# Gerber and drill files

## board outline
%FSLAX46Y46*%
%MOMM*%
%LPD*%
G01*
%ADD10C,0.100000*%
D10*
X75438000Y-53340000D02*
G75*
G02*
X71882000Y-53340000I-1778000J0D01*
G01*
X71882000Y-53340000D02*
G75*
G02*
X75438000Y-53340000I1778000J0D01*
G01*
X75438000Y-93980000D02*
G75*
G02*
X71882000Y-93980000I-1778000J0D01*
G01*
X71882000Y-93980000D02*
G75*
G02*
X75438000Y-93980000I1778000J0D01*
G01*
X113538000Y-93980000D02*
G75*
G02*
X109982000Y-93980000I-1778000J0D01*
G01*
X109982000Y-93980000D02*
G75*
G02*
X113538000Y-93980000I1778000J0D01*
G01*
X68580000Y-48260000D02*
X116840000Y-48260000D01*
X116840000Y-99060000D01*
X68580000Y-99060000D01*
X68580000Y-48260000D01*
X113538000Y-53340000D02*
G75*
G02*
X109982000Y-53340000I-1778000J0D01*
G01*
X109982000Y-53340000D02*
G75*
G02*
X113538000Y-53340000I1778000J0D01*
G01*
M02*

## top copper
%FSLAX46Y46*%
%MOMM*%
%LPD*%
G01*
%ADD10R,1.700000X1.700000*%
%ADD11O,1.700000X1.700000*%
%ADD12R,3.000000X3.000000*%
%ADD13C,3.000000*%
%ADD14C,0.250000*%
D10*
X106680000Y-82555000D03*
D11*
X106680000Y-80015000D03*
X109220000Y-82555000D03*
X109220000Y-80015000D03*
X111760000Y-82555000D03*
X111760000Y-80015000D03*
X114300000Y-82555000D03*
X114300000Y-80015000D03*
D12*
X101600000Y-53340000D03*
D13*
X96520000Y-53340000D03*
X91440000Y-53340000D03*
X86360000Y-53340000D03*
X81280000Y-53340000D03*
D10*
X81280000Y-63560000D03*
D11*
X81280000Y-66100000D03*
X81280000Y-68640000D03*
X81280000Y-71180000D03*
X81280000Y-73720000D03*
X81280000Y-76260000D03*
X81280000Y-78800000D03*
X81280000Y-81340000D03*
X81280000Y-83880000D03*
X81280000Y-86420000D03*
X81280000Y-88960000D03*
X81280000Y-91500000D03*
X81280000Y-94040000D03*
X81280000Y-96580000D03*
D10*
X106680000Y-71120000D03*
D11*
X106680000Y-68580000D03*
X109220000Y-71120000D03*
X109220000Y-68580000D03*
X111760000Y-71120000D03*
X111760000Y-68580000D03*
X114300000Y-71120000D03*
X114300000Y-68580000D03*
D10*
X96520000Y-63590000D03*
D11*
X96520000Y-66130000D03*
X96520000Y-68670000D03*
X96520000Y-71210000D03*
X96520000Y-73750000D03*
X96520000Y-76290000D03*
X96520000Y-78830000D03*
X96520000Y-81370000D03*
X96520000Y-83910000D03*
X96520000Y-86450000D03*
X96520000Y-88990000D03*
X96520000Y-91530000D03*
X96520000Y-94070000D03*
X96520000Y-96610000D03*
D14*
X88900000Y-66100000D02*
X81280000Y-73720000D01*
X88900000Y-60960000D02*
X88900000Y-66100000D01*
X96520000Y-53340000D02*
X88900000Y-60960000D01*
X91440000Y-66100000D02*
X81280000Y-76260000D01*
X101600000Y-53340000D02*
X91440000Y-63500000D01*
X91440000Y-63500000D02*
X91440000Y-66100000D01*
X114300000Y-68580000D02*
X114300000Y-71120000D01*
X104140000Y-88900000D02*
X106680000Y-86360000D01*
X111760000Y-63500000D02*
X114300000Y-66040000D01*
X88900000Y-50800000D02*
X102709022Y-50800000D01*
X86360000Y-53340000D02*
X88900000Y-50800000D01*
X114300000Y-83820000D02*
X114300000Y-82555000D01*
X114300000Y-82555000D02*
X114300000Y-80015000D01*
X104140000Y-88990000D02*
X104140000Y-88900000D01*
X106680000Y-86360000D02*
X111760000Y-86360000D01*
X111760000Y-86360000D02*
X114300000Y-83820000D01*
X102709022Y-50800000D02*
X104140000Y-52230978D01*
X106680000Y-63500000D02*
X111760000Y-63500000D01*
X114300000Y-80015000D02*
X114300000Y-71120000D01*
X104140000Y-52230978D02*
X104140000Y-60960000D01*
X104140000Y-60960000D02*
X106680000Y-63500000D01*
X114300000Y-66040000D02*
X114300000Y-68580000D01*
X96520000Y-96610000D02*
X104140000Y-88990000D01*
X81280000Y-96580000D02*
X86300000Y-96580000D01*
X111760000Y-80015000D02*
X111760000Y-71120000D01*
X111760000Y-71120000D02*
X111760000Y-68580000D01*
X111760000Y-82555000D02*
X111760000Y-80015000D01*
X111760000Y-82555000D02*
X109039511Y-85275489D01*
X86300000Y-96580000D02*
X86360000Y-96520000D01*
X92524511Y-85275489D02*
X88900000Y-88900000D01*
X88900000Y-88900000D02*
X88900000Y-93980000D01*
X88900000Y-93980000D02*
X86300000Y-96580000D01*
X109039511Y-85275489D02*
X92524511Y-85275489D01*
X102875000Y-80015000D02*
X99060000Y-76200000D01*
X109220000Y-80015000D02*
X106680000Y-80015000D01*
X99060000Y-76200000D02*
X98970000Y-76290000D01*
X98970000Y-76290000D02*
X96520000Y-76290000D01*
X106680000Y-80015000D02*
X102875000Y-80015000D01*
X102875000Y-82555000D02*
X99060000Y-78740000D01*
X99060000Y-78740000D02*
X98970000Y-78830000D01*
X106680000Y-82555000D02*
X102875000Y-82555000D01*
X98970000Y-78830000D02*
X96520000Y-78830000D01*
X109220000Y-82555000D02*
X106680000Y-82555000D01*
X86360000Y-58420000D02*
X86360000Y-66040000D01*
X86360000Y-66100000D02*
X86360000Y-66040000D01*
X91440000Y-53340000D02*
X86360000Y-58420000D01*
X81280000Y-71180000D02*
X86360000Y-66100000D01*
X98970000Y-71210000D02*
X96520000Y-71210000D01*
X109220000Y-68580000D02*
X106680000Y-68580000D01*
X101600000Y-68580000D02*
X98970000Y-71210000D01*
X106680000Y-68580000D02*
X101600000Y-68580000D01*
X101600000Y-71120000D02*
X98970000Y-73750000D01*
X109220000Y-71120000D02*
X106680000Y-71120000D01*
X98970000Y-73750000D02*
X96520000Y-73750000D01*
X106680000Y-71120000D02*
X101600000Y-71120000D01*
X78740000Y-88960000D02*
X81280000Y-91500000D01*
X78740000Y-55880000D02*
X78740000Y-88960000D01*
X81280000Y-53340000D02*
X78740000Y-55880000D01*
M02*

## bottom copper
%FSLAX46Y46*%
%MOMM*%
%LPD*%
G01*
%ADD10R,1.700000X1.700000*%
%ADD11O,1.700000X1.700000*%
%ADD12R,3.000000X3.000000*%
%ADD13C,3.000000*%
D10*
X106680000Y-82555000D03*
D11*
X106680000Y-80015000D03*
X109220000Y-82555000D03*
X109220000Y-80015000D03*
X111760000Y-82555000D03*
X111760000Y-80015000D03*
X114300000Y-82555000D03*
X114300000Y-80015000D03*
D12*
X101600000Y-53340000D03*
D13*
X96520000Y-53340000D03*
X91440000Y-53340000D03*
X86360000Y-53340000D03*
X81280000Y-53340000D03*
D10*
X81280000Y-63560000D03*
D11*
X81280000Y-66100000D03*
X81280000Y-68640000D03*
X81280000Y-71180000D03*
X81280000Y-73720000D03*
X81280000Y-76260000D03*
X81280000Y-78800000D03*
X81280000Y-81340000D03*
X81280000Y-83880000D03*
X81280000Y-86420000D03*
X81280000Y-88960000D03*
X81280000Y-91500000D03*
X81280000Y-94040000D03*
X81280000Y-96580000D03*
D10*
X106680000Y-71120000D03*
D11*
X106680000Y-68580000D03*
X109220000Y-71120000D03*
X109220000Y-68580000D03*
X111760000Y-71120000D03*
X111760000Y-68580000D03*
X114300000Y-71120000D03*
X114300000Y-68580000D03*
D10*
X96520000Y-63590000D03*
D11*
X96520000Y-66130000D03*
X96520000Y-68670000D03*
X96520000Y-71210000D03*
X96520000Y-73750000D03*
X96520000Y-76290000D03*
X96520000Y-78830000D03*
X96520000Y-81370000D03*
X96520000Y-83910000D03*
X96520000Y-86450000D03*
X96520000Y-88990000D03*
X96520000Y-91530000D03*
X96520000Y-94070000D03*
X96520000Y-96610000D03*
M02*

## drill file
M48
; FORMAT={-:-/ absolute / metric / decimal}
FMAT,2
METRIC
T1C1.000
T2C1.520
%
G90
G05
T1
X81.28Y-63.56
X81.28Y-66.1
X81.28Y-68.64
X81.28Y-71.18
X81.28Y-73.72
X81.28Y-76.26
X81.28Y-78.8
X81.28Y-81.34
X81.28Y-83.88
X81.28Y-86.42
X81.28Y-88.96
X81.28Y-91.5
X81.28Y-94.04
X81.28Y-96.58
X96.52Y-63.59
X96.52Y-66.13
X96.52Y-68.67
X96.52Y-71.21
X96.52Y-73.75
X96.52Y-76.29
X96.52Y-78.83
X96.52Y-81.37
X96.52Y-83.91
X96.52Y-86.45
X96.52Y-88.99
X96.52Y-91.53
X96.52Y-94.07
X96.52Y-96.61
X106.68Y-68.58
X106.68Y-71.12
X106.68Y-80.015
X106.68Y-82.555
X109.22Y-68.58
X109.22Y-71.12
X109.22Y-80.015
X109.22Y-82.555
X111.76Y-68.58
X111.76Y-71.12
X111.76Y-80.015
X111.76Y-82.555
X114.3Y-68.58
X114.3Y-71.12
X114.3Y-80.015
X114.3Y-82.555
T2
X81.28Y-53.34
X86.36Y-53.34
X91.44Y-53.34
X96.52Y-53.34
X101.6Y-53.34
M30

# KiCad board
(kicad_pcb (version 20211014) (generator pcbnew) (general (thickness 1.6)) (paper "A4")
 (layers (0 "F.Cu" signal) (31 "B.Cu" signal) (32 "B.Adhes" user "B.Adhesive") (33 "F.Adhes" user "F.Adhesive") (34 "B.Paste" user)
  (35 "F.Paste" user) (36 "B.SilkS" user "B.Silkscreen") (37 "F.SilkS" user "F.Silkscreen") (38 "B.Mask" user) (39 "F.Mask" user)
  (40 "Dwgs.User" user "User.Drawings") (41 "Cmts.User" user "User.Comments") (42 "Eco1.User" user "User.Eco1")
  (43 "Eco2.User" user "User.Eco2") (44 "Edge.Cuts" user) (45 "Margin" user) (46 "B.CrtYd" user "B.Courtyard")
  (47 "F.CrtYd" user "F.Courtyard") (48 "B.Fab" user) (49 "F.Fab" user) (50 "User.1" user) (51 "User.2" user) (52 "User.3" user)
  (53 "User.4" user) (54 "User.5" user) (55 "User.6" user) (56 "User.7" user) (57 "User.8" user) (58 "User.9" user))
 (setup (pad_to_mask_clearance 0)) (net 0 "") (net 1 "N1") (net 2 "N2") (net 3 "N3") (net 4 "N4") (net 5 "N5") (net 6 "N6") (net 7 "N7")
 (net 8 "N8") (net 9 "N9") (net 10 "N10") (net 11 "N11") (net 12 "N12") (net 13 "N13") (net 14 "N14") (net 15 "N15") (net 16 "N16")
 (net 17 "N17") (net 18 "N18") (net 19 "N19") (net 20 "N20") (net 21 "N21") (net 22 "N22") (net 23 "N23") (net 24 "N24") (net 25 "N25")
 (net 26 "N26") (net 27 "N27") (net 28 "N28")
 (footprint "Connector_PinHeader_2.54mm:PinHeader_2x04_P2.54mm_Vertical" (layer "F.Cu") (at 106.68 82.555 90)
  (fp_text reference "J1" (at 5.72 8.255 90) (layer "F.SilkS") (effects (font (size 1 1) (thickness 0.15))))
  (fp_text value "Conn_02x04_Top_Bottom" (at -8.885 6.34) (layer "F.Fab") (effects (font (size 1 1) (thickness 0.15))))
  (pad "1" thru_hole rect (at 0 0 90) (size 1.7 1.7) (drill 1) (layers *.Cu *.Mask) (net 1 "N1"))
  (pad "2" thru_hole oval (at 2.54 0 90) (size 1.7 1.7) (drill 1) (layers *.Cu *.Mask) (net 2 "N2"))
  (pad "3" thru_hole oval (at 0 2.54 90) (size 1.7 1.7) (drill 1) (layers *.Cu *.Mask) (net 1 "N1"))
  (pad "4" thru_hole oval (at 2.54 2.54 90) (size 1.7 1.7) (drill 1) (layers *.Cu *.Mask) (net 2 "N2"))
  (pad "5" thru_hole oval (at 0 5.08 90) (size 1.7 1.7) (drill 1) (layers *.Cu *.Mask) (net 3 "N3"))
  (pad "6" thru_hole oval (at 2.54 5.08 90) (size 1.7 1.7) (drill 1) (layers *.Cu *.Mask) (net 3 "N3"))
  (pad "7" thru_hole oval (at 0 7.62 90) (size 1.7 1.7) (drill 1) (layers *.Cu *.Mask) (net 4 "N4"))
  (pad "8" thru_hole oval (at 2.54 7.62 90) (size 1.7 1.7) (drill 1) (layers *.Cu *.Mask) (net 4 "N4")))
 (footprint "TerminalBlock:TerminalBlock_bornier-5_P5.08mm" (layer "F.Cu") (at 101.6 53.34 180)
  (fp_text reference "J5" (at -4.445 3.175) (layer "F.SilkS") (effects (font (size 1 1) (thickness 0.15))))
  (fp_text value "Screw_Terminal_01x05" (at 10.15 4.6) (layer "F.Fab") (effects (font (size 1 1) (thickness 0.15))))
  (pad "1" thru_hole rect (at 0 0 180) (size 3 3) (drill 1.52) (layers *.Cu *.Mask) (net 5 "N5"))
  (pad "2" thru_hole circle (at 5.08 0 180) (size 3 3) (drill 1.52) (layers *.Cu *.Mask) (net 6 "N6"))
  (pad "3" thru_hole circle (at 10.16 0 180) (size 3 3) (drill 1.52) (layers *.Cu *.Mask) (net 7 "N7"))
  (pad "4" thru_hole circle (at 15.24 0 180) (size 3 3) (drill 1.52) (layers *.Cu *.Mask) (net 4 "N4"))
  (pad "5" thru_hole circle (at 20.32 0 180) (size 3 3) (drill 1.52) (layers *.Cu *.Mask) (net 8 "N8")))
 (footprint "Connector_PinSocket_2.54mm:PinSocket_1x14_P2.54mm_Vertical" (layer "F.Cu") (at 81.28 63.56)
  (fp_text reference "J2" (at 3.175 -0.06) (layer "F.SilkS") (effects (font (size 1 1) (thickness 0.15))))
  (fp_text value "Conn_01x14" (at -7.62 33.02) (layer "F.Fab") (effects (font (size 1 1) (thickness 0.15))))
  (pad "1" thru_hole rect (at 0 0) (size 1.7 1.7) (drill 1) (layers *.Cu *.Mask) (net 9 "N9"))
  (pad "2" thru_hole oval (at 0 2.54) (size 1.7 1.7) (drill 1) (layers *.Cu *.Mask) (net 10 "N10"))
  (pad "3" thru_hole oval (at 0 5.08) (size 1.7 1.7) (drill 1) (layers *.Cu *.Mask) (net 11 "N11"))
  (pad "4" thru_hole oval (at 0 7.62) (size 1.7 1.7) (drill 1) (layers *.Cu *.Mask) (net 7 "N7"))
  (pad "5" thru_hole oval (at 0 10.16) (size 1.7 1.7) (drill 1) (layers *.Cu *.Mask) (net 6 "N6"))
  (pad "6" thru_hole oval (at 0 12.7) (size 1.7 1.7) (drill 1) (layers *.Cu *.Mask) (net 5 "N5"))
  (pad "7" thru_hole oval (at 0 15.24) (size 1.7 1.7) (drill 1) (layers *.Cu *.Mask) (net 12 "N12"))
  (pad "8" thru_hole oval (at 0 17.78) (size 1.7 1.7) (drill 1) (layers *.Cu *.Mask) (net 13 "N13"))
  (pad "9" thru_hole oval (at 0 20.32) (size 1.7 1.7) (drill 1) (layers *.Cu *.Mask) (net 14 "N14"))
  (pad "10" thru_hole oval (at 0 22.86) (size 1.7 1.7) (drill 1) (layers *.Cu *.Mask) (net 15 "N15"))
  (pad "11" thru_hole oval (at 0 25.4) (size 1.7 1.7) (drill 1) (layers *.Cu *.Mask) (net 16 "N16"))
  (pad "12" thru_hole oval (at 0 27.94) (size 1.7 1.7) (drill 1) (layers *.Cu *.Mask) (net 8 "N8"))
  (pad "13" thru_hole oval (at 0 30.48) (size 1.7 1.7) (drill 1) (layers *.Cu *.Mask) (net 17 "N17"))
  (pad "14" thru_hole oval (at 0 33.02) (size 1.7 1.7) (drill 1) (layers *.Cu *.Mask) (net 3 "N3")))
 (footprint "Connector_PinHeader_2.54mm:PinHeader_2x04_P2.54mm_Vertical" (layer "F.Cu") (at 106.68 71.12 90)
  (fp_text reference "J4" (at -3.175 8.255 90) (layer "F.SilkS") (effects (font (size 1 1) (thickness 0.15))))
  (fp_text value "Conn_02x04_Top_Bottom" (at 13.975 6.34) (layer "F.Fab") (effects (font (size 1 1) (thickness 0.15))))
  (pad "1" thru_hole rect (at 0 0 90) (size 1.7 1.7) (drill 1) (layers *.Cu *.Mask) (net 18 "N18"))
  (pad "2" thru_hole oval (at 2.54 0 90) (size 1.7 1.7) (drill 1) (layers *.Cu *.Mask) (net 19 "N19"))
  (pad "3" thru_hole oval (at 0 2.54 90) (size 1.7 1.7) (drill 1) (layers *.Cu *.Mask) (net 18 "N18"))
  (pad "4" thru_hole oval (at 2.54 2.54 90) (size 1.7 1.7) (drill 1) (layers *.Cu *.Mask) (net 19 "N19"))
  (pad "5" thru_hole oval (at 0 5.08 90) (size 1.7 1.7) (drill 1) (layers *.Cu *.Mask) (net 3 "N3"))
  (pad "6" thru_hole oval (at 2.54 5.08 90) (size 1.7 1.7) (drill 1) (layers *.Cu *.Mask) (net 3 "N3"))
  (pad "7" thru_hole oval (at 0 7.62 90) (size 1.7 1.7) (drill 1) (layers *.Cu *.Mask) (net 4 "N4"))
  (pad "8" thru_hole oval (at 2.54 7.62 90) (size 1.7 1.7) (drill 1) (layers *.Cu *.Mask) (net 4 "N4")))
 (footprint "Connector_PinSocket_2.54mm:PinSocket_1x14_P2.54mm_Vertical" (layer "F.Cu") (at 96.52 63.59)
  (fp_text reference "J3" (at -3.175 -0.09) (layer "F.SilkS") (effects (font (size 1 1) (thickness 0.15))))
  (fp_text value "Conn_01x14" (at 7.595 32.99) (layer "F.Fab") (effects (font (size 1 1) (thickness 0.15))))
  (pad "1" thru_hole rect (at 0 0) (size 1.7 1.7) (drill 1) (layers *.Cu *.Mask) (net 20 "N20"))
  (pad "2" thru_hole oval (at 0 2.54) (size 1.7 1.7) (drill 1) (layers *.Cu *.Mask) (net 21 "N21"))
  (pad "3" thru_hole oval (at 0 5.08) (size 1.7 1.7) (drill 1) (layers *.Cu *.Mask) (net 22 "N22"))
  (pad "4" thru_hole oval (at 0 7.62) (size 1.7 1.7) (drill 1) (layers *.Cu *.Mask) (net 19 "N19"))
  (pad "5" thru_hole oval (at 0 10.16) (size 1.7 1.7) (drill 1) (layers *.Cu *.Mask) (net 18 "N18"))
  (pad "6" thru_hole oval (at 0 12.7) (size 1.7 1.7) (drill 1) (layers *.Cu *.Mask) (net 2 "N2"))
  (pad "7" thru_hole oval (at 0 15.24) (size 1.7 1.7) (drill 1) (layers *.Cu *.Mask) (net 1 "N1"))
  (pad "8" thru_hole oval (at 0 17.78) (size 1.7 1.7) (drill 1) (layers *.Cu *.Mask) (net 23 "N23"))
  (pad "9" thru_hole oval (at 0 20.32) (size 1.7 1.7) (drill 1) (layers *.Cu *.Mask) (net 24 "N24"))
  (pad "10" thru_hole oval (at 0 22.86) (size 1.7 1.7) (drill 1) (layers *.Cu *.Mask) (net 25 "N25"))
  (pad "11" thru_hole oval (at 0 25.4) (size 1.7 1.7) (drill 1) (layers *.Cu *.Mask) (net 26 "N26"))
  (pad "12" thru_hole oval (at 0 27.94) (size 1.7 1.7) (drill 1) (layers *.Cu *.Mask) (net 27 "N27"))
  (pad "13" thru_hole oval (at 0 30.48) (size 1.7 1.7) (drill 1) (layers *.Cu *.Mask) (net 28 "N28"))
  (pad "14" thru_hole oval (at 0 33.02) (size 1.7 1.7) (drill 1) (layers *.Cu *.Mask) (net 4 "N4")))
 (gr_circle (center 73.66 53.34) (end 73.66 51.562) (layer "Edge.Cuts") (width 0.1) (fill none))
 (gr_circle (center 73.66 93.98) (end 73.66 95.758) (layer "Edge.Cuts") (width 0.1) (fill none))
 (gr_circle (center 111.76 93.98) (end 111.76 95.758) (layer "Edge.Cuts") (width 0.1) (fill none))
 (gr_rect (start 68.58 48.26) (end 116.84 99.06) (layer "Edge.Cuts") (width 0.1) (fill none))
 (gr_circle (center 111.76 53.34) (end 111.76 51.562) (layer "Edge.Cuts") (width 0.1) (fill none))
 (segment (start 88.9 66.1) (end 81.28 73.72) (width 0.25) (layer "F.Cu") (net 6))
 (segment (start 88.9 60.96) (end 88.9 66.1) (width 0.25) (layer "F.Cu") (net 6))
 (segment (start 96.52 53.34) (end 88.9 60.96) (width 0.25) (layer "F.Cu") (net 6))
 (segment (start 91.44 66.1) (end 81.28 76.26) (width 0.25) (layer "F.Cu") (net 5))
 (segment (start 101.6 53.34) (end 91.44 63.5) (width 0.25) (layer "F.Cu") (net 5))
 (segment (start 91.44 63.5) (end 91.44 66.1) (width 0.25) (layer "F.Cu") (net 5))
 (segment (start 114.3 68.58) (end 114.3 71.12) (width 0.25) (layer "F.Cu") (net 4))
 (segment (start 104.14 88.9) (end 106.68 86.36) (width 0.25) (layer "F.Cu") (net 4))
 (segment (start 111.76 63.5) (end 114.3 66.04) (width 0.25) (layer "F.Cu") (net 4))
 (segment (start 88.9 50.8) (end 102.709022 50.8) (width 0.25) (layer "F.Cu") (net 4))
 (segment (start 86.36 53.34) (end 88.9 50.8) (width 0.25) (layer "F.Cu") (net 4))
 (segment (start 114.3 83.82) (end 114.3 82.555) (width 0.25) (layer "F.Cu") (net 4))
 (segment (start 114.3 82.555) (end 114.3 80.015) (width 0.25) (layer "F.Cu") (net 4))
 (segment (start 104.14 88.99) (end 104.14 88.9) (width 0.25) (layer "F.Cu") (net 4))
 (segment (start 106.68 86.36) (end 111.76 86.36) (width 0.25) (layer "F.Cu") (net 4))
 (segment (start 111.76 86.36) (end 114.3 83.82) (width 0.25) (layer "F.Cu") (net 4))
 (segment (start 102.709022 50.8) (end 104.14 52.230978) (width 0.25) (layer "F.Cu") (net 4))
 (segment (start 106.68 63.5) (end 111.76 63.5) (width 0.25) (layer "F.Cu") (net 4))
 (segment (start 114.3 80.015) (end 114.3 71.12) (width 0.25) (layer "F.Cu") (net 4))
 (segment (start 104.14 52.230978) (end 104.14 60.96) (width 0.25) (layer "F.Cu") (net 4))
 (segment (start 104.14 60.96) (end 106.68 63.5) (width 0.25) (layer "F.Cu") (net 4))
 (segment (start 114.3 66.04) (end 114.3 68.58) (width 0.25) (layer "F.Cu") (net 4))
 (segment (start 96.52 96.61) (end 104.14 88.99) (width 0.25) (layer "F.Cu") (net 4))
 (segment (start 81.28 96.58) (end 86.3 96.58) (width 0.25) (layer "F.Cu") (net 3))
 (segment (start 111.76 80.015) (end 111.76 71.12) (width 0.25) (layer "F.Cu") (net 3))
 (segment (start 111.76 71.12) (end 111.76 68.58) (width 0.25) (layer "F.Cu") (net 3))
 (segment (start 111.76 82.555) (end 111.76 80.015) (width 0.25) (layer "F.Cu") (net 3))
 (segment (start 111.76 82.555) (end 109.039511 85.275489) (width 0.25) (layer "F.Cu") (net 3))
 (segment (start 86.3 96.58) (end 86.36 96.52) (width 0.25) (layer "F.Cu") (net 3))
 (segment (start 92.524511 85.275489) (end 88.9 88.9) (width 0.25) (layer "F.Cu") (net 3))
 (segment (start 88.9 88.9) (end 88.9 93.98) (width 0.25) (layer "F.Cu") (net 3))
 (segment (start 88.9 93.98) (end 86.3 96.58) (width 0.25) (layer "F.Cu") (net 3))
 (segment (start 109.039511 85.275489) (end 92.524511 85.275489) (width 0.25) (layer "F.Cu") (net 3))
 (segment (start 102.875 80.015) (end 99.06 76.2) (width 0.25) (layer "F.Cu") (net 2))
 (segment (start 109.22 80.015) (end 106.68 80.015) (width 0.25) (layer "F.Cu") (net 2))
 (segment (start 99.06 76.2) (end 98.97 76.29) (width 0.25) (layer "F.Cu") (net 2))
 (segment (start 98.97 76.29) (end 96.52 76.29) (width 0.25) (layer "F.Cu") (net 2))
 (segment (start 106.68 80.015) (end 102.875 80.015) (width 0.25) (layer "F.Cu") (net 2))
 (segment (start 102.875 82.555) (end 99.06 78.74) (width 0.25) (layer "F.Cu") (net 1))
 (segment (start 99.06 78.74) (end 98.97 78.83) (width 0.25) (layer "F.Cu") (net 1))
 (segment (start 106.68 82.555) (end 102.875 82.555) (width 0.25) (layer "F.Cu") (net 1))
 (segment (start 98.97 78.83) (end 96.52 78.83) (width 0.25) (layer "F.Cu") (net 1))
 (segment (start 109.22 82.555) (end 106.68 82.555) (width 0.25) (layer "F.Cu") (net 1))
 (segment (start 86.36 58.42) (end 86.36 66.04) (width 0.25) (layer "F.Cu") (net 7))
 (segment (start 86.36 66.1) (end 86.36 66.04) (width 0.25) (layer "F.Cu") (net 7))
 (segment (start 91.44 53.34) (end 86.36 58.42) (width 0.25) (layer "F.Cu") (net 7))
 (segment (start 81.28 71.18) (end 86.36 66.1) (width 0.25) (layer "F.Cu") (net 7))
 (segment (start 98.97 71.21) (end 96.52 71.21) (width 0.25) (layer "F.Cu") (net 19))
 (segment (start 109.22 68.58) (end 106.68 68.58) (width 0.25) (layer "F.Cu") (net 19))
 (segment (start 101.6 68.58) (end 98.97 71.21) (width 0.25) (layer "F.Cu") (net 19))
 (segment (start 106.68 68.58) (end 101.6 68.58) (width 0.25) (layer "F.Cu") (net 19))
 (segment (start 101.6 71.12) (end 98.97 73.75) (width 0.25) (layer "F.Cu") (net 18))
 (segment (start 109.22 71.12) (end 106.68 71.12) (width 0.25) (layer "F.Cu") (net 18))
 (segment (start 98.97 73.75) (end 96.52 73.75) (width 0.25) (layer "F.Cu") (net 18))
 (segment (start 106.68 71.12) (end 101.6 71.12) (width 0.25) (layer "F.Cu") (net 18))
 (segment (start 78.74 88.96) (end 81.28 91.5) (width 0.25) (layer "F.Cu") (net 8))
 (segment (start 78.74 55.88) (end 78.74 88.96) (width 0.25) (layer "F.Cu") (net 8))
 (segment (start 81.28 53.34) (end 78.74 55.88) (width 0.25) (layer "F.Cu") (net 8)))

